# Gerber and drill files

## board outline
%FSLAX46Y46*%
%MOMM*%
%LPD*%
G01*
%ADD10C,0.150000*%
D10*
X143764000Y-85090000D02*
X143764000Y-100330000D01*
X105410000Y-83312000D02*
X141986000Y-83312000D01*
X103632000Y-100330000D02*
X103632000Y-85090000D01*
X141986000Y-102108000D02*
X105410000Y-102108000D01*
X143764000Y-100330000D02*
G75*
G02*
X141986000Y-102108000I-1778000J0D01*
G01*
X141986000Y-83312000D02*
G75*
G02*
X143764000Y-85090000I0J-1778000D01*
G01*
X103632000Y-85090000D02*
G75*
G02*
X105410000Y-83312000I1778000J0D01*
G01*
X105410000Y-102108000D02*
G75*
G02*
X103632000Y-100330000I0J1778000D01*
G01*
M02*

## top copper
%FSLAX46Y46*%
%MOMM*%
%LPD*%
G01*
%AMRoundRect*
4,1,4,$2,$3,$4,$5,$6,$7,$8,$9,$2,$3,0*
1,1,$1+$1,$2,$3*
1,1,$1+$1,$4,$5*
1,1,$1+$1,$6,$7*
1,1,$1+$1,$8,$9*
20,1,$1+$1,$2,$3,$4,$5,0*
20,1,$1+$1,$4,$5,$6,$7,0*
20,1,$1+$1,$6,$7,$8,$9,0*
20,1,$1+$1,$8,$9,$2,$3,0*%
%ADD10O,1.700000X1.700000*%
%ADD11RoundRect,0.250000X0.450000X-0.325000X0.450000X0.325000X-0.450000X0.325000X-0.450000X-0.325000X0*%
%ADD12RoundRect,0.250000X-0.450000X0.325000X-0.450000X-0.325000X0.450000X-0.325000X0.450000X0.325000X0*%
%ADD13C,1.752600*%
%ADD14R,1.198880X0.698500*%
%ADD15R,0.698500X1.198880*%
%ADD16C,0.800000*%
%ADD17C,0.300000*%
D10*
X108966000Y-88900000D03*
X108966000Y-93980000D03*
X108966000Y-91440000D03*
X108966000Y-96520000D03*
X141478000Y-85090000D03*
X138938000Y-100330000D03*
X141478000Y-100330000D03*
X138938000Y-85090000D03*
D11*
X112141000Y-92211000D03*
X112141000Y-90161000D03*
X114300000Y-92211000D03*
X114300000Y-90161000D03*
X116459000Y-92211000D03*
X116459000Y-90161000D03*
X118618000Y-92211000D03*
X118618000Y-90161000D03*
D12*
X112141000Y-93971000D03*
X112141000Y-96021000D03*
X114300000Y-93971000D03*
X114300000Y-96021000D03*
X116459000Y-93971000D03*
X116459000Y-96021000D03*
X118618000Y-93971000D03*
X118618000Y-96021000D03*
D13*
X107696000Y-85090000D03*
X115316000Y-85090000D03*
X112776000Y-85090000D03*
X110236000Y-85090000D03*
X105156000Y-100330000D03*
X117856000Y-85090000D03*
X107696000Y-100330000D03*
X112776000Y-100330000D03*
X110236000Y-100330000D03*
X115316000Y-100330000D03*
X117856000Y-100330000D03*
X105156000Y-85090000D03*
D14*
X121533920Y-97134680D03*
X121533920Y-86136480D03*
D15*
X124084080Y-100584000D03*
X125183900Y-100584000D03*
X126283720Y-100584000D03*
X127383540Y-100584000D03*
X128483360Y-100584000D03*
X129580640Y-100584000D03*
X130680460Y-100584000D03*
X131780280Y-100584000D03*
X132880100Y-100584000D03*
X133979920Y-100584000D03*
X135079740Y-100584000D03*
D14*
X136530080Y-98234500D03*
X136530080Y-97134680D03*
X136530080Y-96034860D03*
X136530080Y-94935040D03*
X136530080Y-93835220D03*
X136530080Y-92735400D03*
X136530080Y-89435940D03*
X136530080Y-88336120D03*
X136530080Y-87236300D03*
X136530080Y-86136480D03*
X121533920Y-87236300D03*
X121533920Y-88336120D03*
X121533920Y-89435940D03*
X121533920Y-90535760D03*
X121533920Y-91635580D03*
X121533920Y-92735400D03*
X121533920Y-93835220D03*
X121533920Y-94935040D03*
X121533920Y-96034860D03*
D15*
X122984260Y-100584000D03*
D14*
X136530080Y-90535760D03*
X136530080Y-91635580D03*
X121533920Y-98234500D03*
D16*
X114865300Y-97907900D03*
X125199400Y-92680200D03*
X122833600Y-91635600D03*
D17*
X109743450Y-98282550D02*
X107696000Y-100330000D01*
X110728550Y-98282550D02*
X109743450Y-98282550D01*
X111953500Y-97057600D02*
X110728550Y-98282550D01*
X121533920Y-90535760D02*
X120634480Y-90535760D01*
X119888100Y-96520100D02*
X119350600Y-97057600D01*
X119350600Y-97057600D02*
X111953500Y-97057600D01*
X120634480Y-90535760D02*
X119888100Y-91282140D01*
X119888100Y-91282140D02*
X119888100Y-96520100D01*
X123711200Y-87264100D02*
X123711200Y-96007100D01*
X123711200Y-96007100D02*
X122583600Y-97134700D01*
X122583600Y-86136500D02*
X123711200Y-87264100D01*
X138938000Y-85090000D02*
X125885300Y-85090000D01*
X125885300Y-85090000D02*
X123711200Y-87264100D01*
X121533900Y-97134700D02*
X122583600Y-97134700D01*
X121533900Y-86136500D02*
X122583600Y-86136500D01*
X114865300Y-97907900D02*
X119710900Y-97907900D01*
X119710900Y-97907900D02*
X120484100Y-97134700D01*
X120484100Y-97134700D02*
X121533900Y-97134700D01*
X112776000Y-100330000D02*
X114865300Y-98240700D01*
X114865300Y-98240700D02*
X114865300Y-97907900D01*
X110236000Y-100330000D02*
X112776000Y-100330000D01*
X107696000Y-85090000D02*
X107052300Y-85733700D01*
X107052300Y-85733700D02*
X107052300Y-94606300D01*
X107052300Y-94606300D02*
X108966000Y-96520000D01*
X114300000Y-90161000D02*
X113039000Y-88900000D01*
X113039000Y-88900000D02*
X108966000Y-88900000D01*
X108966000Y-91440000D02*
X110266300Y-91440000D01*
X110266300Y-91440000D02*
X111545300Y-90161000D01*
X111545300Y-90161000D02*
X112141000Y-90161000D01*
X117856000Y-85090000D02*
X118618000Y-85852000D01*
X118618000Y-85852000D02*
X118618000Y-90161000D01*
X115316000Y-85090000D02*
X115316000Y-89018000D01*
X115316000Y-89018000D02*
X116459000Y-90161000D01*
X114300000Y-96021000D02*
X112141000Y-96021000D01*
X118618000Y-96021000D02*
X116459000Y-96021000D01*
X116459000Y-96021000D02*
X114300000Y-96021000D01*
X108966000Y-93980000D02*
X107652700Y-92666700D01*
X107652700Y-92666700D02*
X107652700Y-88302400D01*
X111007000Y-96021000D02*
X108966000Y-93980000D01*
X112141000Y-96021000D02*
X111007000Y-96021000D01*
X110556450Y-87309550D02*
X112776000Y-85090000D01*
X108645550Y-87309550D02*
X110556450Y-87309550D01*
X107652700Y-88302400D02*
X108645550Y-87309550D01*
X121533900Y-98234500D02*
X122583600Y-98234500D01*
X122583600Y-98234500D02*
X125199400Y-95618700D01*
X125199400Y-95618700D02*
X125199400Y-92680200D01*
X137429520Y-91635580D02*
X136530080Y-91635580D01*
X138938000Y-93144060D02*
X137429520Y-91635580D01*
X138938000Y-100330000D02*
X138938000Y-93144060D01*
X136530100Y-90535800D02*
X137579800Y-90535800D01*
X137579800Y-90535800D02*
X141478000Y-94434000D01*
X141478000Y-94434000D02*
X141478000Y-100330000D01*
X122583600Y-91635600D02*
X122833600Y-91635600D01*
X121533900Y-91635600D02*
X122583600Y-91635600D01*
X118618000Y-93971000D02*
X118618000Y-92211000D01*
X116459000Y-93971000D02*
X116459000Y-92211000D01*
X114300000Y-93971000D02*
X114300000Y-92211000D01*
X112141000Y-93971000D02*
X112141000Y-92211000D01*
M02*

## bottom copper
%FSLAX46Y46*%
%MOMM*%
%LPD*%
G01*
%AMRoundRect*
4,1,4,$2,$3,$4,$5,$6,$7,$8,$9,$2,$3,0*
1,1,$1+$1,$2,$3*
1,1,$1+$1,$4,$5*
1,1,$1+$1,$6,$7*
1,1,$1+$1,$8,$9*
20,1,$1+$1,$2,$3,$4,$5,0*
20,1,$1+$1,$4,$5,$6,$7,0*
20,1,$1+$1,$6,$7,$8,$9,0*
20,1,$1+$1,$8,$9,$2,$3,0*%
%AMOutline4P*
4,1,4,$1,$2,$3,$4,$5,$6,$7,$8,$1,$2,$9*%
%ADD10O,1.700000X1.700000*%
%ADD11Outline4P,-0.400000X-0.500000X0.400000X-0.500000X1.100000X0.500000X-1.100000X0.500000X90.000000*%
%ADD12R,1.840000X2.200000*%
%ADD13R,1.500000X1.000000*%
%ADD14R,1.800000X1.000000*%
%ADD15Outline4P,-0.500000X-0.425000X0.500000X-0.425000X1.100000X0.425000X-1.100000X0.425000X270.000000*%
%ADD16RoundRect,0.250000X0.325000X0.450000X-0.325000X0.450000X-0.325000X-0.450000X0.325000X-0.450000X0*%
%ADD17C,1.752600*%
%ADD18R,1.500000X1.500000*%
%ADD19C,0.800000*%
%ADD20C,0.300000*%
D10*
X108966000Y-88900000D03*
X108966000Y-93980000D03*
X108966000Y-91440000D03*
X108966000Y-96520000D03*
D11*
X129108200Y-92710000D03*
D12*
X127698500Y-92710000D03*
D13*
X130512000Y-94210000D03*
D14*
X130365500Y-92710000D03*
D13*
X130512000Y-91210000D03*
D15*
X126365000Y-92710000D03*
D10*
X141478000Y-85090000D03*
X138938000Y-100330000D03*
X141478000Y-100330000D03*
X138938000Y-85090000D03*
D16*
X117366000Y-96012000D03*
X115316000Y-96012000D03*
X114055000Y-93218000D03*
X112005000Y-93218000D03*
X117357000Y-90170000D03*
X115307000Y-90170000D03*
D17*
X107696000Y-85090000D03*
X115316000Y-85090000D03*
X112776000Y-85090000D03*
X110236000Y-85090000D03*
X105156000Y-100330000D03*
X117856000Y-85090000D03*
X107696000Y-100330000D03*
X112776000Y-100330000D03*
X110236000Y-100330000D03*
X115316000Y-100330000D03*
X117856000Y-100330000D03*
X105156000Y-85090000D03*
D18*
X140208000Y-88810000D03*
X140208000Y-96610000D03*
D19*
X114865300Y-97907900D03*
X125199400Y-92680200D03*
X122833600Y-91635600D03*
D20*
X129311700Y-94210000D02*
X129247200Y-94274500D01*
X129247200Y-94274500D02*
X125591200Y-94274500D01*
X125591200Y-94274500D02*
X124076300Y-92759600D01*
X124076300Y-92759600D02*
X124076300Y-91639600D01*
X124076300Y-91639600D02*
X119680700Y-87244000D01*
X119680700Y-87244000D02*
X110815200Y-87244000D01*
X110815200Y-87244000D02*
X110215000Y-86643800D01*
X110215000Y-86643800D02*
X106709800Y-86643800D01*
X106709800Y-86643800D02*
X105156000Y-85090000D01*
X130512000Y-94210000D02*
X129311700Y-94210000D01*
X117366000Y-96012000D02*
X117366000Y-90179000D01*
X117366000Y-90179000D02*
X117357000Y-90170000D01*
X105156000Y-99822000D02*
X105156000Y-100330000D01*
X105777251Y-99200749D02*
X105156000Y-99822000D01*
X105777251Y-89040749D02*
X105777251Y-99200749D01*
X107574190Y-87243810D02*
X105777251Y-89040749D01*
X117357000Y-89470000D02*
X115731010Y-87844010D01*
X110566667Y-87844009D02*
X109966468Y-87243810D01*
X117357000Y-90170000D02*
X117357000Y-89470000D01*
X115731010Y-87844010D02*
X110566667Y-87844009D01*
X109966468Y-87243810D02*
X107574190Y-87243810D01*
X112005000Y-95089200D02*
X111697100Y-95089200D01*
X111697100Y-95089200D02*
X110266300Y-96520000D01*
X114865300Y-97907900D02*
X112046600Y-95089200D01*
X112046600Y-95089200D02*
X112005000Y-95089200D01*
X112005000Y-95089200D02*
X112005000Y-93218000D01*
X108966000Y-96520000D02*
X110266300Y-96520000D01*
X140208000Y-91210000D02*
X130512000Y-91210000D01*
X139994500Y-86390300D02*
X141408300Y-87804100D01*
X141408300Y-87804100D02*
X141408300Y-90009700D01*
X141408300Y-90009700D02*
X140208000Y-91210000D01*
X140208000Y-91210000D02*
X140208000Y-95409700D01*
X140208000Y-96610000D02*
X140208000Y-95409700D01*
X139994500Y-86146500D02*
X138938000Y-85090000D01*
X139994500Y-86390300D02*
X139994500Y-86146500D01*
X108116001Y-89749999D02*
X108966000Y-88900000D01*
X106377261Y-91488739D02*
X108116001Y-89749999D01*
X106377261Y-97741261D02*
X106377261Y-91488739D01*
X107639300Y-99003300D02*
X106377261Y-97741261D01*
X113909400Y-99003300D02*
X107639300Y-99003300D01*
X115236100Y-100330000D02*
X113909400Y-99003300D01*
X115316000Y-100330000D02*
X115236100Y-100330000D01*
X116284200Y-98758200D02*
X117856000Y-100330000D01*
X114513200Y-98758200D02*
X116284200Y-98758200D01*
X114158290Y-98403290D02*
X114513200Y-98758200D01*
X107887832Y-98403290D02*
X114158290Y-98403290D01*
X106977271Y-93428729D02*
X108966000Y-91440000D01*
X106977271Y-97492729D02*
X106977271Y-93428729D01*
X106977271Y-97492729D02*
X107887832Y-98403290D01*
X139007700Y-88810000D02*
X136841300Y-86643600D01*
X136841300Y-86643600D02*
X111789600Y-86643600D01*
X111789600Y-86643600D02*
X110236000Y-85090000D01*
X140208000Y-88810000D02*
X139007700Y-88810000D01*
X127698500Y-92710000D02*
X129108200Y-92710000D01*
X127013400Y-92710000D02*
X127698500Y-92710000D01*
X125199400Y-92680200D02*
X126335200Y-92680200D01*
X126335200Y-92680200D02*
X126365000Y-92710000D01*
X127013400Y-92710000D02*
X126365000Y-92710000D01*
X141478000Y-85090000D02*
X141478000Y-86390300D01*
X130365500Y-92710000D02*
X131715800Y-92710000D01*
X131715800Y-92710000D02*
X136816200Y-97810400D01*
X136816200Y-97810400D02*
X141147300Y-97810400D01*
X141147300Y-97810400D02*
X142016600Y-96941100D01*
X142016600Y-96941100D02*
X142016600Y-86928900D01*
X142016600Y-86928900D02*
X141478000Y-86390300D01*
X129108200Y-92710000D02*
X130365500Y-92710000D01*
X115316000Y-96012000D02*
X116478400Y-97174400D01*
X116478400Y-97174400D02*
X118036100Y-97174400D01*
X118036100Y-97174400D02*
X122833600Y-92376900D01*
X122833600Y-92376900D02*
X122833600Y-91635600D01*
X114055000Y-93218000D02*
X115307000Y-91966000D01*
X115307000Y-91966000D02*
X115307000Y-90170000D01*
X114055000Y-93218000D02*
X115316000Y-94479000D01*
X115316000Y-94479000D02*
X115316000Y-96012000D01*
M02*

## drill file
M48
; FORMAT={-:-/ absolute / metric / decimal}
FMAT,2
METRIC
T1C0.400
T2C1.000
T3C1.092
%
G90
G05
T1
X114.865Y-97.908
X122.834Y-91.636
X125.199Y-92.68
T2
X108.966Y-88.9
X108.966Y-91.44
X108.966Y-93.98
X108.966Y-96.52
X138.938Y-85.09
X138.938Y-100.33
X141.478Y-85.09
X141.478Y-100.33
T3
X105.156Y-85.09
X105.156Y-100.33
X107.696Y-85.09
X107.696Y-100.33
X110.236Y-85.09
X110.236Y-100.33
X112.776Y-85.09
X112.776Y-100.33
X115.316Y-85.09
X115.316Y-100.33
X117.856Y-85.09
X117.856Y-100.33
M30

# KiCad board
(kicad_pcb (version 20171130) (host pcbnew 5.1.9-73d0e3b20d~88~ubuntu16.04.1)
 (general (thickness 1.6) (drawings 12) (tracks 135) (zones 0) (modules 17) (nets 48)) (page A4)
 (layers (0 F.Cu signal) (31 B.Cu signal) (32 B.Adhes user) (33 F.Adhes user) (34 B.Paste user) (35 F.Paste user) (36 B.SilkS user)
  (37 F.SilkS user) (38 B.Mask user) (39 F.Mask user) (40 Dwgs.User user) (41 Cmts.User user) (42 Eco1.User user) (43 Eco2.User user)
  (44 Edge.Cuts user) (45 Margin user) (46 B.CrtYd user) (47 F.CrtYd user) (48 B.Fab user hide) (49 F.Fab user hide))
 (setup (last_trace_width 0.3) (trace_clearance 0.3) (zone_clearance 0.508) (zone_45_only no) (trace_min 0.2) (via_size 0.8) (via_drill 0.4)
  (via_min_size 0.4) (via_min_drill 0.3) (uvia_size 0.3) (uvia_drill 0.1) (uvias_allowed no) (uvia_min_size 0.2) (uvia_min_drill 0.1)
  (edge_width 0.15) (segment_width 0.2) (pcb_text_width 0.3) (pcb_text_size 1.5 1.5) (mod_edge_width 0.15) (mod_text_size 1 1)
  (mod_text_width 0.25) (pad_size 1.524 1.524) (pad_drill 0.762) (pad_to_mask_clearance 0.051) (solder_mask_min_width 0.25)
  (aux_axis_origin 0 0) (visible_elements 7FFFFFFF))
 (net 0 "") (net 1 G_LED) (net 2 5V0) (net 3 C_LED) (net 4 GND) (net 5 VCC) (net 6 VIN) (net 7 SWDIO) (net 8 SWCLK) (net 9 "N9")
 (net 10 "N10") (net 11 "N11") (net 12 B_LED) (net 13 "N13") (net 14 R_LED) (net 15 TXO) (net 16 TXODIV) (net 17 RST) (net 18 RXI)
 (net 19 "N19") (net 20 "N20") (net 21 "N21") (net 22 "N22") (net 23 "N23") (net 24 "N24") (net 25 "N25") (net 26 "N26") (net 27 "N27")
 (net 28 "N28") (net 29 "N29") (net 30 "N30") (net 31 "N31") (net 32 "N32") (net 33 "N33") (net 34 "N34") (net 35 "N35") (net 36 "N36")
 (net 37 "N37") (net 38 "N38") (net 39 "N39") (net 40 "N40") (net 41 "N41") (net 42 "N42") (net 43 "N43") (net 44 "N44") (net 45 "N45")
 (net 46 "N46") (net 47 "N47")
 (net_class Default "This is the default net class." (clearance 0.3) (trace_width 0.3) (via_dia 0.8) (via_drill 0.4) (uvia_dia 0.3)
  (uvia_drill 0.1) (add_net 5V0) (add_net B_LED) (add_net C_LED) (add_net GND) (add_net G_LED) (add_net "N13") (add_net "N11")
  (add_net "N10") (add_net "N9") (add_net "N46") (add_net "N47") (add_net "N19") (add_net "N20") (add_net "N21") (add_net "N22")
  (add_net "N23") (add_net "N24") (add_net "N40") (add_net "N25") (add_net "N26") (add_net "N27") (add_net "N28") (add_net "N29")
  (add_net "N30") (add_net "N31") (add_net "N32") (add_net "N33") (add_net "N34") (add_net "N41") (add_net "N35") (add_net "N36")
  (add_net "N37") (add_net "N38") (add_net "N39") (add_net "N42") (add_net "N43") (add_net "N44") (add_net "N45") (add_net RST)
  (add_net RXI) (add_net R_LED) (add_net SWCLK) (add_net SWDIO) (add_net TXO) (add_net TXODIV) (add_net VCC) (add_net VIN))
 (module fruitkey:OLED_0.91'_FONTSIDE (layer F.Cu) (at 108.966 92.71)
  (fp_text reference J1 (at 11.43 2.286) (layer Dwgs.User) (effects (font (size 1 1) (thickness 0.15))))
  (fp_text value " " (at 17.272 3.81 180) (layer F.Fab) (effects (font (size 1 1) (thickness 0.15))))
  (pad 4 thru_hole oval (at 0 -3.81) (size 1.7 1.7) (drill 1) (layers *.Cu *.Mask) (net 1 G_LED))
  (pad 2 thru_hole oval (at 0 1.27) (size 1.7 1.7) (drill 1) (layers *.Cu *.Mask) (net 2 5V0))
  (pad 3 thru_hole oval (at 0 -1.27) (size 1.7 1.7) (drill 1) (layers *.Cu *.Mask) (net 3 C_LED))
  (pad 1 thru_hole oval (at 0 3.81) (size 1.7 1.7) (drill 1) (layers *.Cu *.Mask) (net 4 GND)))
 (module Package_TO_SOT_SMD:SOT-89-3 (layer B.Cu) (at 129.032 92.71 180)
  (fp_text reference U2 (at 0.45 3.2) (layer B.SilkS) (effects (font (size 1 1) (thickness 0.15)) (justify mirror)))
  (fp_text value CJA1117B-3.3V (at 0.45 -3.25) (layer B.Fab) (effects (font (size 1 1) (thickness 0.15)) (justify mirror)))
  (pad 2 smd trapezoid (at -0.0762 0 90) (size 1.5 1) (rect_delta 0 -0.7) (layers B.Cu B.Paste B.Mask) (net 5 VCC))
  (pad 2 smd rect (at 1.3335 0 270) (size 2.2 1.84) (layers B.Cu B.Paste B.Mask) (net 5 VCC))
  (pad 3 smd rect (at -1.48 -1.5 270) (size 1 1.5) (layers B.Cu B.Paste B.Mask) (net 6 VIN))
  (pad 2 smd rect (at -1.3335 0 270) (size 1 1.8) (layers B.Cu B.Paste B.Mask) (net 5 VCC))
  (pad 1 smd rect (at -1.48 1.5 270) (size 1 1.5) (layers B.Cu B.Paste B.Mask) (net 4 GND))
  (pad 2 smd trapezoid (at 2.667 0 270) (size 1.6 0.85) (rect_delta 0 -0.6) (layers B.Cu B.Paste B.Mask) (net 5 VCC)))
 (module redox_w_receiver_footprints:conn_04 (layer B.Cu) (at 137.668 85.09 180)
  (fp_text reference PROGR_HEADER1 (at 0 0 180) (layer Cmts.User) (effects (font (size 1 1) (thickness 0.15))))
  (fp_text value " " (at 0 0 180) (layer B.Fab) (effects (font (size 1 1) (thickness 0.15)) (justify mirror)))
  (pad 1 thru_hole oval (at -3.81 0 90) (size 1.7 1.7) (drill 1) (layers *.Cu *.Mask) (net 5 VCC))
  (pad 3 thru_hole oval (at -1.27 -15.24 90) (size 1.7 1.7) (drill 1) (layers *.Cu *.Mask) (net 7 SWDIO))
  (pad 4 thru_hole oval (at -3.81 -15.24 90) (size 1.7 1.7) (drill 1) (layers *.Cu *.Mask) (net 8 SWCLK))
  (pad 2 thru_hole oval (at -1.27 0 90) (size 1.7 1.7) (drill 1) (layers *.Cu *.Mask) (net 4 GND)))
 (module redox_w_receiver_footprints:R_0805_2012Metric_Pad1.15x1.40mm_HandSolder (layer F.Cu) (at 112.141 91.186 90)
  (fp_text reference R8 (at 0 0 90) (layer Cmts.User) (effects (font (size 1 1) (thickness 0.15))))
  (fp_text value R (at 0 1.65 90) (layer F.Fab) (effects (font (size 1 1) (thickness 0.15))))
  (pad 1 smd roundrect (at -1.025 0 90) (size 1.15 1.4) (layers F.Cu F.Paste F.Mask) (roundrect_rratio 0.217391) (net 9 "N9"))
  (pad 2 smd roundrect (at 1.025 0 90) (size 1.15 1.4) (layers F.Cu F.Paste F.Mask) (roundrect_rratio 0.217391) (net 3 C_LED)))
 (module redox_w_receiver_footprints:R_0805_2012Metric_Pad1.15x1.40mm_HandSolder (layer F.Cu) (at 114.3 91.186 90)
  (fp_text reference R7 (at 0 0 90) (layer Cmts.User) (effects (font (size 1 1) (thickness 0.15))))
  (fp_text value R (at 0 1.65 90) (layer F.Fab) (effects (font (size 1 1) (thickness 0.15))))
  (pad 1 smd roundrect (at -1.025 0 90) (size 1.15 1.4) (layers F.Cu F.Paste F.Mask) (roundrect_rratio 0.217391) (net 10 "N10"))
  (pad 2 smd roundrect (at 1.025 0 90) (size 1.15 1.4) (layers F.Cu F.Paste F.Mask) (roundrect_rratio 0.217391) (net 1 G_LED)))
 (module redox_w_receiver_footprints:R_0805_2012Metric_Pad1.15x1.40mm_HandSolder (layer F.Cu) (at 116.459 91.186 90)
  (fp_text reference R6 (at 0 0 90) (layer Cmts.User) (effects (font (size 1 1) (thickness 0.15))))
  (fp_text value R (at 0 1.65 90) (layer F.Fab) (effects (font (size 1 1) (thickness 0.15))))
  (pad 1 smd roundrect (at -1.025 0 90) (size 1.15 1.4) (layers F.Cu F.Paste F.Mask) (roundrect_rratio 0.217391) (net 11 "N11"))
  (pad 2 smd roundrect (at 1.025 0 90) (size 1.15 1.4) (layers F.Cu F.Paste F.Mask) (roundrect_rratio 0.217391) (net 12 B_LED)))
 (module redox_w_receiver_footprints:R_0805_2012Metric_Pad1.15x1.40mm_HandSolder (layer F.Cu) (at 118.618 91.186 90)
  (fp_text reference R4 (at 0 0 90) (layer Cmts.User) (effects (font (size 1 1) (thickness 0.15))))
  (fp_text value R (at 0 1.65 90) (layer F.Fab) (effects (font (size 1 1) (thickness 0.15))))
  (pad 1 smd roundrect (at -1.025 0 90) (size 1.15 1.4) (layers F.Cu F.Paste F.Mask) (roundrect_rratio 0.217391) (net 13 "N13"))
  (pad 2 smd roundrect (at 1.025 0 90) (size 1.15 1.4) (layers F.Cu F.Paste F.Mask) (roundrect_rratio 0.217391) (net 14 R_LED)))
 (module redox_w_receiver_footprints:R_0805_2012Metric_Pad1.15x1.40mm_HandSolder (layer B.Cu) (at 116.341 96.012 180)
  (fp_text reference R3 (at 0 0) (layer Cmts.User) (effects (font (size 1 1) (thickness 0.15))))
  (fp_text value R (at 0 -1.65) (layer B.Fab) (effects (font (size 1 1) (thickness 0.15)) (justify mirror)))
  (pad 1 smd roundrect (at -1.025 0 180) (size 1.15 1.4) (layers B.Cu B.Paste B.Mask) (roundrect_rratio 0.217391) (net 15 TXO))
  (pad 2 smd roundrect (at 1.025 0 180) (size 1.15 1.4) (layers B.Cu B.Paste B.Mask) (roundrect_rratio 0.217391) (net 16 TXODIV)))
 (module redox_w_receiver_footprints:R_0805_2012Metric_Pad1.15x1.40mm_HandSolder (layer B.Cu) (at 113.03 93.218 180)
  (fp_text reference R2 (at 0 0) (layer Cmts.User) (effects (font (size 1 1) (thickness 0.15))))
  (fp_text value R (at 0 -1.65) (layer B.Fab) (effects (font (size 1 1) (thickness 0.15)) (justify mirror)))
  (pad 1 smd roundrect (at -1.025 0 180) (size 1.15 1.4) (layers B.Cu B.Paste B.Mask) (roundrect_rratio 0.217391) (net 16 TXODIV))
  (pad 2 smd roundrect (at 1.025 0 180) (size 1.15 1.4) (layers B.Cu B.Paste B.Mask) (roundrect_rratio 0.217391) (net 4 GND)))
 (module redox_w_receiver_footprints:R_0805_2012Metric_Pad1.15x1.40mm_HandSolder (layer B.Cu) (at 116.332 90.17 180)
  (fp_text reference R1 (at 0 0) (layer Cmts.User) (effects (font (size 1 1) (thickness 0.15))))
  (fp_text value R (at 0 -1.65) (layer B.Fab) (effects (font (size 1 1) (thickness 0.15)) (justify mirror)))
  (pad 1 smd roundrect (at -1.025 0 180) (size 1.15 1.4) (layers B.Cu B.Paste B.Mask) (roundrect_rratio 0.217391) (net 15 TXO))
  (pad 2 smd roundrect (at 1.025 0 180) (size 1.15 1.4) (layers B.Cu B.Paste B.Mask) (roundrect_rratio 0.217391) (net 16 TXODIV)))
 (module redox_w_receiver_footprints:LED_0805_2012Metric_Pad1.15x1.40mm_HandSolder (layer F.Cu) (at 112.141 94.996 270)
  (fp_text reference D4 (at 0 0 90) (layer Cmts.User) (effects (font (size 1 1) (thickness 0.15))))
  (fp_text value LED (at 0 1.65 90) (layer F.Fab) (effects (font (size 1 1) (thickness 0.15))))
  (pad 1 smd roundrect (at -1.025 0 270) (size 1.15 1.4) (layers F.Cu F.Paste F.Mask) (roundrect_rratio 0.217391) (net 9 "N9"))
  (pad 2 smd roundrect (at 1.025 0 270) (size 1.15 1.4) (layers F.Cu F.Paste F.Mask) (roundrect_rratio 0.217391) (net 2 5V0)))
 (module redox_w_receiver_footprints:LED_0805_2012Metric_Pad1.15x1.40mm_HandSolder (layer F.Cu) (at 114.3 94.996 270)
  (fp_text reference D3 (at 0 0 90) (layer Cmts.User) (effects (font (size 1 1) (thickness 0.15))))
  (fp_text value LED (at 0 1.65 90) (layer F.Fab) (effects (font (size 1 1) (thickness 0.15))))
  (pad 1 smd roundrect (at -1.025 0 270) (size 1.15 1.4) (layers F.Cu F.Paste F.Mask) (roundrect_rratio 0.217391) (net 10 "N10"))
  (pad 2 smd roundrect (at 1.025 0 270) (size 1.15 1.4) (layers F.Cu F.Paste F.Mask) (roundrect_rratio 0.217391) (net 2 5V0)))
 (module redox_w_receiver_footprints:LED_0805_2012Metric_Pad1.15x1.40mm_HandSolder (layer F.Cu) (at 116.459 94.996 270)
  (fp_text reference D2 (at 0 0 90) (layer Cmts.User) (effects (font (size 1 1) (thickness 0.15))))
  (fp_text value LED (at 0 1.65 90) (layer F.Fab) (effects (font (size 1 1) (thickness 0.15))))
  (pad 1 smd roundrect (at -1.025 0 270) (size 1.15 1.4) (layers F.Cu F.Paste F.Mask) (roundrect_rratio 0.217391) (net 11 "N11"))
  (pad 2 smd roundrect (at 1.025 0 270) (size 1.15 1.4) (layers F.Cu F.Paste F.Mask) (roundrect_rratio 0.217391) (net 2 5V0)))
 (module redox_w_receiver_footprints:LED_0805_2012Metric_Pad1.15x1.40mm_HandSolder (layer F.Cu) (at 118.618 94.996 270)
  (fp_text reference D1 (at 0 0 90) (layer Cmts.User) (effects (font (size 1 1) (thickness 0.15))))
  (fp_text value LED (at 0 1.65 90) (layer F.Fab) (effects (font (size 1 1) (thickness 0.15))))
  (pad 1 smd roundrect (at -1.025 0 270) (size 1.15 1.4) (layers F.Cu F.Paste F.Mask) (roundrect_rratio 0.217391) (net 13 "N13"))
  (pad 2 smd roundrect (at 1.025 0 270) (size 1.15 1.4) (layers F.Cu F.Paste F.Mask) (roundrect_rratio 0.217391) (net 2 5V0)))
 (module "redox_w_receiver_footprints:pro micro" (layer F.Cu) (at 119.126 92.71 90)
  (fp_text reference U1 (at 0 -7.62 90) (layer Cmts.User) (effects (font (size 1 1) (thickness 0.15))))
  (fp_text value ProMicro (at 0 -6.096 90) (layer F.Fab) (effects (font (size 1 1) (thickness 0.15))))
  (pad GND thru_hole circle (at 7.62 -11.43) (size 1.7526 1.7526) (drill 1.0922) (layers *.Cu *.SilkS *.Mask) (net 4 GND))
  (pad F4 thru_hole circle (at 7.62 -3.81) (size 1.7526 1.7526) (drill 1.0922) (layers *.Cu *.SilkS *.Mask) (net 12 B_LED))
  (pad VCC thru_hole circle (at 7.62 -6.35) (size 1.7526 1.7526) (drill 1.0922) (layers *.Cu *.SilkS *.Mask) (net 2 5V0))
  (pad RST thru_hole circle (at 7.62 -8.89) (size 1.7526 1.7526) (drill 1.0922) (layers *.Cu *.SilkS *.Mask) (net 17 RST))
  (pad D3 thru_hole circle (at -7.62 -13.97 180) (size 1.7526 1.7526) (drill 1.0922) (layers *.Cu *.SilkS *.Mask) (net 15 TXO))
  (pad F5 thru_hole circle (at 7.62 -1.27) (size 1.7526 1.7526) (drill 1.0922) (layers *.Cu *.SilkS *.Mask) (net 14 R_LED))
  (pad D2 thru_hole circle (at -7.62 -11.43) (size 1.7526 1.7526) (drill 1.0922) (layers *.Cu *.SilkS *.Mask) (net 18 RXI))
  (pad GND thru_hole circle (at -7.62 -6.35) (size 1.7526 1.7526) (drill 1.0922) (layers *.Cu *.SilkS *.Mask) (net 4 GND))
  (pad GND thru_hole circle (at -7.62 -8.89) (size 1.7526 1.7526) (drill 1.0922) (layers *.Cu *.SilkS *.Mask) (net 4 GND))
  (pad D1 thru_hole circle (at -7.62 -3.81) (size 1.7526 1.7526) (drill 1.0922) (layers *.Cu *.SilkS *.Mask) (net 1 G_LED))
  (pad D0 thru_hole circle (at -7.62 -1.27) (size 1.7526 1.7526) (drill 1.0922) (layers *.Cu *.SilkS *.Mask) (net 3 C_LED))
  (pad RAW thru_hole circle (at 7.62 -13.97) (size 1.7526 1.7526) (drill 1.0922) (layers *.Cu *.SilkS *.Mask) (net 6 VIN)))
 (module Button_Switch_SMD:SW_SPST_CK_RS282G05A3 (layer B.Cu) (at 140.208 92.71 270)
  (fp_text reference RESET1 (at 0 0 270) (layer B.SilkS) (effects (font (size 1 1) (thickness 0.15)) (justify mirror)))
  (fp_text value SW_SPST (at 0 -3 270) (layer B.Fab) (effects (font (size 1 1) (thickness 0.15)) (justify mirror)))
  (pad 1 smd rect (at -3.9 0 270) (size 1.5 1.5) (layers B.Cu B.Paste B.Mask) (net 17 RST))
  (pad 2 smd rect (at 3.9 0 270) (size 1.5 1.5) (layers B.Cu B.Paste B.Mask) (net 4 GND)))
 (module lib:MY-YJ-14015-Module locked (layer F.Cu) (at 129.032 100.584)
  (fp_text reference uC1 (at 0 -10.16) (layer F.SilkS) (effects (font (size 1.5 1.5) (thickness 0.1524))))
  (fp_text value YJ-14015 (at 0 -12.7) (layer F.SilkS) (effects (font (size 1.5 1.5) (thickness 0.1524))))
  (pad 11 smd rect (at -7.49808 -3.44932 90) (size 0.6985 1.19888) (layers F.Cu F.Paste F.Mask) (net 4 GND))
  (pad 1 smd rect (at -7.49808 -14.44752 90) (size 0.6985 1.19888) (layers F.Cu F.Paste F.Mask) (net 4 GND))
  (pad 14 smd rect (at -4.94792 0 90) (size 1.19888 0.6985) (layers F.Cu F.Paste F.Mask) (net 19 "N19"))
  (pad 15 smd rect (at -3.8481 0 90) (size 1.19888 0.6985) (layers F.Cu F.Paste F.Mask) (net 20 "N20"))
  (pad 16 smd rect (at -2.74828 0 90) (size 1.19888 0.6985) (layers F.Cu F.Paste F.Mask) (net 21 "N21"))
  (pad 17 smd rect (at -1.64846 0 90) (size 1.19888 0.6985) (layers F.Cu F.Paste F.Mask) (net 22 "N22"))
  (pad 18 smd rect (at -0.54864 0 90) (size 1.19888 0.6985) (layers F.Cu F.Paste F.Mask) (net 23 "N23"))
  (pad 19 smd rect (at 0.54864 0 90) (size 1.19888 0.6985) (layers F.Cu F.Paste F.Mask) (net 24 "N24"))
  (pad 20 smd rect (at 1.64846 0 90) (size 1.19888 0.6985) (layers F.Cu F.Paste F.Mask) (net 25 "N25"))
  (pad 21 smd rect (at 2.74828 0 90) (size 1.19888 0.6985) (layers F.Cu F.Paste F.Mask) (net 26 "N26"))
  (pad 22 smd rect (at 3.8481 0 90) (size 1.19888 0.6985) (layers F.Cu F.Paste F.Mask) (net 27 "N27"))
  (pad 23 smd rect (at 4.94792 0 90) (size 1.19888 0.6985) (layers F.Cu F.Paste F.Mask) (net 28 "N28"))
  (pad 24 smd rect (at 6.04774 0 90) (size 1.19888 0.6985) (layers F.Cu F.Paste F.Mask) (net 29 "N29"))
  (pad 25 smd rect (at 7.49808 -2.3495 90) (size 0.6985 1.19888) (layers F.Cu F.Paste F.Mask) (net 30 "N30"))
  (pad 26 smd rect (at 7.49808 -3.44932 90) (size 0.6985 1.19888) (layers F.Cu F.Paste F.Mask) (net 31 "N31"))
  (pad 27 smd rect (at 7.49808 -4.54914 90) (size 0.6985 1.19888) (layers F.Cu F.Paste F.Mask) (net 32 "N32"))
  (pad 28 smd rect (at 7.49808 -5.64896 90) (size 0.6985 1.19888) (layers F.Cu F.Paste F.Mask) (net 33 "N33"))
  (pad 29 smd rect (at 7.49808 -6.74878 90) (size 0.6985 1.19888) (layers F.Cu F.Paste F.Mask) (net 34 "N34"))
  (pad 30 smd rect (at 7.49808 -7.8486 90) (size 0.6985 1.19888) (layers F.Cu F.Paste F.Mask) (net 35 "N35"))
  (pad 33 smd rect (at 7.49808 -11.14806 90) (size 0.6985 1.19888) (layers F.Cu F.Paste F.Mask) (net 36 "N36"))
  (pad 34 smd rect (at 7.49808 -12.24788 90) (size 0.6985 1.19888) (layers F.Cu F.Paste F.Mask) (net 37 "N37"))
  (pad 35 smd rect (at 7.49808 -13.3477 90) (size 0.6985 1.19888) (layers F.Cu F.Paste F.Mask) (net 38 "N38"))
  (pad 36 smd rect (at 7.49808 -14.44752 90) (size 0.6985 1.19888) (layers F.Cu F.Paste F.Mask) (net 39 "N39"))
  (pad 2 smd rect (at -7.49808 -13.3477 90) (size 0.6985 1.19888) (layers F.Cu F.Paste F.Mask) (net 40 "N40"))
  (pad 3 smd rect (at -7.49808 -12.24788 90) (size 0.6985 1.19888) (layers F.Cu F.Paste F.Mask) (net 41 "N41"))
  (pad 4 smd rect (at -7.49808 -11.14806 90) (size 0.6985 1.19888) (layers F.Cu F.Paste F.Mask) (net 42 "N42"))
  (pad 5 smd rect (at -7.49808 -10.04824 90) (size 0.6985 1.19888) (layers F.Cu F.Paste F.Mask) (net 18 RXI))
  (pad 6 smd rect (at -7.49808 -8.94842 90) (size 0.6985 1.19888) (layers F.Cu F.Paste F.Mask) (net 16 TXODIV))
  (pad 7 smd rect (at -7.49808 -7.8486 90) (size 0.6985 1.19888) (layers F.Cu F.Paste F.Mask) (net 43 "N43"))
  (pad 8 smd rect (at -7.49808 -6.74878 90) (size 0.6985 1.19888) (layers F.Cu F.Paste F.Mask) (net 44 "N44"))
  (pad 9 smd rect (at -7.49808 -5.64896 90) (size 0.6985 1.19888) (layers F.Cu F.Paste F.Mask) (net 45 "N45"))
  (pad 10 smd rect (at -7.49808 -4.54914 90) (size 0.6985 1.19888) (layers F.Cu F.Paste F.Mask) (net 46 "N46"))
  (pad 13 smd rect (at -6.04774 0 90) (size 1.19888 0.6985) (layers F.Cu F.Paste F.Mask) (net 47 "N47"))
  (pad 32 smd rect (at 7.49808 -10.04824 90) (size 0.6985 1.19888) (layers F.Cu F.Paste F.Mask) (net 8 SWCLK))
  (pad 31 smd rect (at 7.49808 -8.94842 90) (size 0.6985 1.19888) (layers F.Cu F.Paste F.Mask) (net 7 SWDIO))
  (pad 12 smd rect (at -7.49808 -2.3495 90) (size 0.6985 1.19888) (layers F.Cu F.Paste F.Mask) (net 5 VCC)))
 (gr_line (start 143.764 85.09) (end 143.764 100.33) (layer Edge.Cuts) (width 0.15))
 (gr_line (start 105.41 83.312) (end 141.986 83.312) (layer Edge.Cuts) (width 0.15))
 (gr_line (start 103.632 100.33) (end 103.632 85.09) (layer Edge.Cuts) (width 0.15))
 (gr_line (start 141.986 102.108) (end 105.41 102.108) (layer Edge.Cuts) (width 0.15))
 (gr_arc (start 141.986 100.33) (end 141.986 102.108) (angle -90) (layer Edge.Cuts) (width 0.15))
 (gr_arc (start 141.986 85.09) (end 143.764 85.09) (angle -90) (layer Edge.Cuts) (width 0.15))
 (gr_arc (start 105.41 85.09) (end 105.41 83.312) (angle -90) (layer Edge.Cuts) (width 0.15))
 (gr_arc (start 105.41 100.33) (end 103.632 100.33) (angle -90) (layer Edge.Cuts) (width 0.15))
 (segment (start 129.3117 94.21) (end 129.2472 94.2745) (width 0.3) (layer B.Cu) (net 6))
 (segment (start 129.2472 94.2745) (end 125.5912 94.2745) (width 0.3) (layer B.Cu) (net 6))
 (segment (start 125.5912 94.2745) (end 124.0763 92.7596) (width 0.3) (layer B.Cu) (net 6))
 (segment (start 124.0763 92.7596) (end 124.0763 91.6396) (width 0.3) (layer B.Cu) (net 6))
 (segment (start 124.0763 91.6396) (end 119.6807 87.244) (width 0.3) (layer B.Cu) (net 6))
 (segment (start 119.6807 87.244) (end 110.8152 87.244) (width 0.3) (layer B.Cu) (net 6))
 (segment (start 110.8152 87.244) (end 110.215 86.6438) (width 0.3) (layer B.Cu) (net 6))
 (segment (start 110.215 86.6438) (end 106.7098 86.6438) (width 0.3) (layer B.Cu) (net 6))
 (segment (start 106.7098 86.6438) (end 105.156 85.09) (width 0.3) (layer B.Cu) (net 6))
 (segment (start 130.512 94.21) (end 129.3117 94.21) (width 0.3) (layer B.Cu) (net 6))
 (segment (start 117.366 96.012) (end 117.366 90.179) (width 0.3) (layer B.Cu) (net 15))
 (segment (start 117.366 90.179) (end 117.357 90.17) (width 0.3) (layer B.Cu) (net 15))
 (segment (start 105.156 99.822) (end 105.156 100.33) (width 0.3) (layer B.Cu) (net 15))
 (segment (start 105.777251 99.200749) (end 105.156 99.822) (width 0.3) (layer B.Cu) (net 15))
 (segment (start 105.777251 89.040749) (end 105.777251 99.200749) (width 0.3) (layer B.Cu) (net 15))
 (segment (start 107.57419 87.24381) (end 105.777251 89.040749) (width 0.3) (layer B.Cu) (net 15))
 (segment (start 117.357 89.47) (end 115.73101 87.84401) (width 0.3) (layer B.Cu) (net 15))
 (segment (start 110.566667 87.844009) (end 109.966468 87.24381) (width 0.3) (layer B.Cu) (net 15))
 (segment (start 117.357 90.17) (end 117.357 89.47) (width 0.3) (layer B.Cu) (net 15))
 (segment (start 115.73101 87.84401) (end 110.566667 87.844009) (width 0.3) (layer B.Cu) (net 15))
 (segment (start 109.966468 87.24381) (end 107.57419 87.24381) (width 0.3) (layer B.Cu) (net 15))
 (segment (start 109.74345 98.28255) (end 107.696 100.33) (width 0.3) (layer F.Cu) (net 18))
 (segment (start 110.72855 98.28255) (end 109.74345 98.28255) (width 0.3) (layer F.Cu) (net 18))
 (segment (start 111.9535 97.0576) (end 110.72855 98.28255) (width 0.3) (layer F.Cu) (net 18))
 (segment (start 121.53392 90.53576) (end 120.63448 90.53576) (width 0.3) (layer F.Cu) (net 18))
 (segment (start 119.8881 96.5201) (end 119.3506 97.0576) (width 0.3) (layer F.Cu) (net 18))
 (segment (start 119.3506 97.0576) (end 111.9535 97.0576) (width 0.3) (layer F.Cu) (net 18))
 (segment (start 120.63448 90.53576) (end 119.8881 91.28214) (width 0.3) (layer F.Cu) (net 18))
 (segment (start 119.8881 91.28214) (end 119.8881 96.5201) (width 0.3) (layer F.Cu) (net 18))
 (segment (start 123.7112 87.2641) (end 123.7112 96.0071) (width 0.3) (layer F.Cu) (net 4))
 (segment (start 123.7112 96.0071) (end 122.5836 97.1347) (width 0.3) (layer F.Cu) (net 4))
 (segment (start 122.5836 86.1365) (end 123.7112 87.2641) (width 0.3) (layer F.Cu) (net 4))
 (segment (start 138.938 85.09) (end 125.8853 85.09) (width 0.3) (layer F.Cu) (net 4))
 (segment (start 125.8853 85.09) (end 123.7112 87.2641) (width 0.3) (layer F.Cu) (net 4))
 (segment (start 121.5339 97.1347) (end 122.5836 97.1347) (width 0.3) (layer F.Cu) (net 4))
 (segment (start 121.5339 86.1365) (end 122.5836 86.1365) (width 0.3) (layer F.Cu) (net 4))
 (segment (start 112.005 95.0892) (end 111.6971 95.0892) (width 0.3) (layer B.Cu) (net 4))
 (segment (start 111.6971 95.0892) (end 110.2663 96.52) (width 0.3) (layer B.Cu) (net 4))
 (segment (start 114.8653 97.9079) (end 112.0466 95.0892) (width 0.3) (layer B.Cu) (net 4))
 (segment (start 112.0466 95.0892) (end 112.005 95.0892) (width 0.3) (layer B.Cu) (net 4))
 (segment (start 112.005 95.0892) (end 112.005 93.218) (width 0.3) (layer B.Cu) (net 4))
 (segment (start 108.966 96.52) (end 110.2663 96.52) (width 0.3) (layer B.Cu) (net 4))
 (segment (start 114.8653 97.9079) (end 119.7109 97.9079) (width 0.3) (layer F.Cu) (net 4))
 (segment (start 119.7109 97.9079) (end 120.4841 97.1347) (width 0.3) (layer F.Cu) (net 4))
 (segment (start 120.4841 97.1347) (end 121.5339 97.1347) (width 0.3) (layer F.Cu) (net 4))
 (segment (start 112.776 100.33) (end 114.8653 98.2407) (width 0.3) (layer F.Cu) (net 4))
 (segment (start 114.8653 98.2407) (end 114.8653 97.9079) (width 0.3) (layer F.Cu) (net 4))
 (segment (start 110.236 100.33) (end 112.776 100.33) (width 0.3) (layer F.Cu) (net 4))
 (segment (start 140.208 91.21) (end 130.512 91.21) (width 0.3) (layer B.Cu) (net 4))
 (segment (start 139.9945 86.3903) (end 141.4083 87.8041) (width 0.3) (layer B.Cu) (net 4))
 (segment (start 141.4083 87.8041) (end 141.4083 90.0097) (width 0.3) (layer B.Cu) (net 4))
 (segment (start 141.4083 90.0097) (end 140.208 91.21) (width 0.3) (layer B.Cu) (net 4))
 (segment (start 140.208 91.21) (end 140.208 95.4097) (width 0.3) (layer B.Cu) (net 4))
 (segment (start 140.208 96.61) (end 140.208 95.4097) (width 0.3) (layer B.Cu) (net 4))
 (segment (start 107.696 85.09) (end 107.0523 85.7337) (width 0.3) (layer F.Cu) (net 4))
 (segment (start 107.0523 85.7337) (end 107.0523 94.6063) (width 0.3) (layer F.Cu) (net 4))
 (segment (start 107.0523 94.6063) (end 108.966 96.52) (width 0.3) (layer F.Cu) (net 4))
 (via (at 114.8653 97.9079) (size 0.8) (layers F.Cu B.Cu) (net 4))
 (segment (start 139.9945 86.1465) (end 138.938 85.09) (width 0.3) (layer B.Cu) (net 4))
 (segment (start 139.9945 86.3903) (end 139.9945 86.1465) (width 0.3) (layer B.Cu) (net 4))
 (segment (start 114.3 90.161) (end 113.039 88.9) (width 0.3) (layer F.Cu) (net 1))
 (segment (start 113.039 88.9) (end 108.966 88.9) (width 0.3) (layer F.Cu) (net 1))
 (segment (start 108.116001 89.749999) (end 108.966 88.9) (width 0.3) (layer B.Cu) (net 1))
 (segment (start 106.377261 91.488739) (end 108.116001 89.749999) (width 0.3) (layer B.Cu) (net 1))
 (segment (start 106.377261 97.741261) (end 106.377261 91.488739) (width 0.3) (layer B.Cu) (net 1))
 (segment (start 107.6393 99.0033) (end 106.377261 97.741261) (width 0.3) (layer B.Cu) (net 1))
 (segment (start 113.9094 99.0033) (end 107.6393 99.0033) (width 0.3) (layer B.Cu) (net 1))
 (segment (start 115.2361 100.33) (end 113.9094 99.0033) (width 0.3) (layer B.Cu) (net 1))
 (segment (start 115.316 100.33) (end 115.2361 100.33) (width 0.3) (layer B.Cu) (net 1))
 (segment (start 108.966 91.44) (end 110.2663 91.44) (width 0.3) (layer F.Cu) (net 3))
 (segment (start 110.2663 91.44) (end 111.5453 90.161) (width 0.3) (layer F.Cu) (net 3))
 (segment (start 111.5453 90.161) (end 112.141 90.161) (width 0.3) (layer F.Cu) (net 3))
 (segment (start 116.2842 98.7582) (end 117.856 100.33) (width 0.3) (layer B.Cu) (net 3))
 (segment (start 114.5132 98.7582) (end 116.2842 98.7582) (width 0.3) (layer B.Cu) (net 3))
 (segment (start 114.15829 98.40329) (end 114.5132 98.7582) (width 0.3) (layer B.Cu) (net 3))
 (segment (start 107.887832 98.40329) (end 114.15829 98.40329) (width 0.3) (layer B.Cu) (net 3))
 (segment (start 106.977271 93.428729) (end 108.966 91.44) (width 0.3) (layer B.Cu) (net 3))
 (segment (start 106.977271 97.492729) (end 106.977271 93.428729) (width 0.3) (layer B.Cu) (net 3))
 (segment (start 106.977271 97.492729) (end 107.887832 98.40329) (width 0.3) (layer B.Cu) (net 3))
 (segment (start 117.856 85.09) (end 118.618 85.852) (width 0.3) (layer F.Cu) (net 14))
 (segment (start 118.618 85.852) (end 118.618 90.161) (width 0.3) (layer F.Cu) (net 14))
 (segment (start 115.316 85.09) (end 115.316 89.018) (width 0.3) (layer F.Cu) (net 12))
 (segment (start 115.316 89.018) (end 116.459 90.161) (width 0.3) (layer F.Cu) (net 12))
 (segment (start 114.3 96.021) (end 112.141 96.021) (width 0.3) (layer F.Cu) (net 2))
 (segment (start 118.618 96.021) (end 116.459 96.021) (width 0.3) (layer F.Cu) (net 2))
 (segment (start 116.459 96.021) (end 114.3 96.021) (width 0.3) (layer F.Cu) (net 2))
 (segment (start 108.966 93.98) (end 107.6527 92.6667) (width 0.3) (layer F.Cu) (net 2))
 (segment (start 107.6527 92.6667) (end 107.6527 88.3024) (width 0.3) (layer F.Cu) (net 2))
 (segment (start 111.007 96.021) (end 108.966 93.98) (width 0.3) (layer F.Cu) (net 2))
 (segment (start 112.141 96.021) (end 111.007 96.021) (width 0.3) (layer F.Cu) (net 2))
 (segment (start 110.55645 87.30955) (end 112.776 85.09) (width 0.3) (layer F.Cu) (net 2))
 (segment (start 108.64555 87.30955) (end 110.55645 87.30955) (width 0.3) (layer F.Cu) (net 2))
 (segment (start 107.6527 88.3024) (end 108.64555 87.30955) (width 0.3) (layer F.Cu) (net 2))
 (segment (start 139.0077 88.81) (end 136.8413 86.6436) (width 0.3) (layer B.Cu) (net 17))
 (segment (start 136.8413 86.6436) (end 111.7896 86.6436) (width 0.3) (layer B.Cu) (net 17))
 (segment (start 111.7896 86.6436) (end 110.236 85.09) (width 0.3) (layer B.Cu) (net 17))
 (segment (start 140.208 88.81) (end 139.0077 88.81) (width 0.3) (layer B.Cu) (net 17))
 (segment (start 127.6985 92.71) (end 129.1082 92.71) (width 0.3) (layer B.Cu) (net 5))
 (segment (start 127.0134 92.71) (end 127.6985 92.71) (width 0.3) (layer B.Cu) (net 5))
 (segment (start 121.5339 98.2345) (end 122.5836 98.2345) (width 0.3) (layer F.Cu) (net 5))
 (segment (start 125.1994 92.6802) (end 126.3352 92.6802) (width 0.3) (layer B.Cu) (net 5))
 (segment (start 126.3352 92.6802) (end 126.365 92.71) (width 0.3) (layer B.Cu) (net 5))
 (segment (start 122.5836 98.2345) (end 125.1994 95.6187) (width 0.3) (layer F.Cu) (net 5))
 (segment (start 125.1994 95.6187) (end 125.1994 92.6802) (width 0.3) (layer F.Cu) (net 5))
 (segment (start 127.0134 92.71) (end 126.365 92.71) (width 0.3) (layer B.Cu) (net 5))
 (segment (start 141.478 85.09) (end 141.478 86.3903) (width 0.3) (layer B.Cu) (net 5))
 (segment (start 130.3655 92.71) (end 131.7158 92.71) (width 0.3) (layer B.Cu) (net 5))
 (segment (start 131.7158 92.71) (end 136.8162 97.8104) (width 0.3) (layer B.Cu) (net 5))
 (segment (start 136.8162 97.8104) (end 141.1473 97.8104) (width 0.3) (layer B.Cu) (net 5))
 (segment (start 141.1473 97.8104) (end 142.0166 96.9411) (width 0.3) (layer B.Cu) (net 5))
 (segment (start 142.0166 96.9411) (end 142.0166 86.9289) (width 0.3) (layer B.Cu) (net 5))
 (segment (start 142.0166 86.9289) (end 141.478 86.3903) (width 0.3) (layer B.Cu) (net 5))
 (segment (start 129.1082 92.71) (end 130.3655 92.71) (width 0.3) (layer B.Cu) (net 5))
 (via (at 125.1994 92.6802) (size 0.8) (layers F.Cu B.Cu) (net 5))
 (segment (start 137.42952 91.63558) (end 136.53008 91.63558) (width 0.3) (layer F.Cu) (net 7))
 (segment (start 138.938 93.14406) (end 137.42952 91.63558) (width 0.3) (layer F.Cu) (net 7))
 (segment (start 138.938 100.33) (end 138.938 93.14406) (width 0.3) (layer F.Cu) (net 7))
 (segment (start 136.5301 90.5358) (end 137.5798 90.5358) (width 0.3) (layer F.Cu) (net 8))
 (segment (start 137.5798 90.5358) (end 141.478 94.434) (width 0.3) (layer F.Cu) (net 8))
 (segment (start 141.478 94.434) (end 141.478 100.33) (width 0.3) (layer F.Cu) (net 8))
 (segment (start 122.5836 91.6356) (end 122.8336 91.6356) (width 0.3) (layer F.Cu) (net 16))
 (segment (start 115.316 96.012) (end 116.4784 97.1744) (width 0.3) (layer B.Cu) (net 16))
 (segment (start 116.4784 97.1744) (end 118.0361 97.1744) (width 0.3) (layer B.Cu) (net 16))
 (segment (start 118.0361 97.1744) (end 122.8336 92.3769) (width 0.3) (layer B.Cu) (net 16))
 (segment (start 122.8336 92.3769) (end 122.8336 91.6356) (width 0.3) (layer B.Cu) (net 16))
 (segment (start 121.5339 91.6356) (end 122.5836 91.6356) (width 0.3) (layer F.Cu) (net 16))
 (segment (start 114.055 93.218) (end 115.307 91.966) (width 0.3) (layer B.Cu) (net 16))
 (segment (start 115.307 91.966) (end 115.307 90.17) (width 0.3) (layer B.Cu) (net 16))
 (segment (start 114.055 93.218) (end 115.316 94.479) (width 0.3) (layer B.Cu) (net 16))
 (segment (start 115.316 94.479) (end 115.316 96.012) (width 0.3) (layer B.Cu) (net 16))
 (via (at 122.8336 91.6356) (size 0.8) (layers F.Cu B.Cu) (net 16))
 (segment (start 118.618 93.971) (end 118.618 92.211) (width 0.3) (layer F.Cu) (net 13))
 (segment (start 116.459 93.971) (end 116.459 92.211) (width 0.3) (layer F.Cu) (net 11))
 (segment (start 114.3 93.971) (end 114.3 92.211) (width 0.3) (layer F.Cu) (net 10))
 (segment (start 112.141 93.971) (end 112.141 92.211) (width 0.3) (layer F.Cu) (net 9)))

